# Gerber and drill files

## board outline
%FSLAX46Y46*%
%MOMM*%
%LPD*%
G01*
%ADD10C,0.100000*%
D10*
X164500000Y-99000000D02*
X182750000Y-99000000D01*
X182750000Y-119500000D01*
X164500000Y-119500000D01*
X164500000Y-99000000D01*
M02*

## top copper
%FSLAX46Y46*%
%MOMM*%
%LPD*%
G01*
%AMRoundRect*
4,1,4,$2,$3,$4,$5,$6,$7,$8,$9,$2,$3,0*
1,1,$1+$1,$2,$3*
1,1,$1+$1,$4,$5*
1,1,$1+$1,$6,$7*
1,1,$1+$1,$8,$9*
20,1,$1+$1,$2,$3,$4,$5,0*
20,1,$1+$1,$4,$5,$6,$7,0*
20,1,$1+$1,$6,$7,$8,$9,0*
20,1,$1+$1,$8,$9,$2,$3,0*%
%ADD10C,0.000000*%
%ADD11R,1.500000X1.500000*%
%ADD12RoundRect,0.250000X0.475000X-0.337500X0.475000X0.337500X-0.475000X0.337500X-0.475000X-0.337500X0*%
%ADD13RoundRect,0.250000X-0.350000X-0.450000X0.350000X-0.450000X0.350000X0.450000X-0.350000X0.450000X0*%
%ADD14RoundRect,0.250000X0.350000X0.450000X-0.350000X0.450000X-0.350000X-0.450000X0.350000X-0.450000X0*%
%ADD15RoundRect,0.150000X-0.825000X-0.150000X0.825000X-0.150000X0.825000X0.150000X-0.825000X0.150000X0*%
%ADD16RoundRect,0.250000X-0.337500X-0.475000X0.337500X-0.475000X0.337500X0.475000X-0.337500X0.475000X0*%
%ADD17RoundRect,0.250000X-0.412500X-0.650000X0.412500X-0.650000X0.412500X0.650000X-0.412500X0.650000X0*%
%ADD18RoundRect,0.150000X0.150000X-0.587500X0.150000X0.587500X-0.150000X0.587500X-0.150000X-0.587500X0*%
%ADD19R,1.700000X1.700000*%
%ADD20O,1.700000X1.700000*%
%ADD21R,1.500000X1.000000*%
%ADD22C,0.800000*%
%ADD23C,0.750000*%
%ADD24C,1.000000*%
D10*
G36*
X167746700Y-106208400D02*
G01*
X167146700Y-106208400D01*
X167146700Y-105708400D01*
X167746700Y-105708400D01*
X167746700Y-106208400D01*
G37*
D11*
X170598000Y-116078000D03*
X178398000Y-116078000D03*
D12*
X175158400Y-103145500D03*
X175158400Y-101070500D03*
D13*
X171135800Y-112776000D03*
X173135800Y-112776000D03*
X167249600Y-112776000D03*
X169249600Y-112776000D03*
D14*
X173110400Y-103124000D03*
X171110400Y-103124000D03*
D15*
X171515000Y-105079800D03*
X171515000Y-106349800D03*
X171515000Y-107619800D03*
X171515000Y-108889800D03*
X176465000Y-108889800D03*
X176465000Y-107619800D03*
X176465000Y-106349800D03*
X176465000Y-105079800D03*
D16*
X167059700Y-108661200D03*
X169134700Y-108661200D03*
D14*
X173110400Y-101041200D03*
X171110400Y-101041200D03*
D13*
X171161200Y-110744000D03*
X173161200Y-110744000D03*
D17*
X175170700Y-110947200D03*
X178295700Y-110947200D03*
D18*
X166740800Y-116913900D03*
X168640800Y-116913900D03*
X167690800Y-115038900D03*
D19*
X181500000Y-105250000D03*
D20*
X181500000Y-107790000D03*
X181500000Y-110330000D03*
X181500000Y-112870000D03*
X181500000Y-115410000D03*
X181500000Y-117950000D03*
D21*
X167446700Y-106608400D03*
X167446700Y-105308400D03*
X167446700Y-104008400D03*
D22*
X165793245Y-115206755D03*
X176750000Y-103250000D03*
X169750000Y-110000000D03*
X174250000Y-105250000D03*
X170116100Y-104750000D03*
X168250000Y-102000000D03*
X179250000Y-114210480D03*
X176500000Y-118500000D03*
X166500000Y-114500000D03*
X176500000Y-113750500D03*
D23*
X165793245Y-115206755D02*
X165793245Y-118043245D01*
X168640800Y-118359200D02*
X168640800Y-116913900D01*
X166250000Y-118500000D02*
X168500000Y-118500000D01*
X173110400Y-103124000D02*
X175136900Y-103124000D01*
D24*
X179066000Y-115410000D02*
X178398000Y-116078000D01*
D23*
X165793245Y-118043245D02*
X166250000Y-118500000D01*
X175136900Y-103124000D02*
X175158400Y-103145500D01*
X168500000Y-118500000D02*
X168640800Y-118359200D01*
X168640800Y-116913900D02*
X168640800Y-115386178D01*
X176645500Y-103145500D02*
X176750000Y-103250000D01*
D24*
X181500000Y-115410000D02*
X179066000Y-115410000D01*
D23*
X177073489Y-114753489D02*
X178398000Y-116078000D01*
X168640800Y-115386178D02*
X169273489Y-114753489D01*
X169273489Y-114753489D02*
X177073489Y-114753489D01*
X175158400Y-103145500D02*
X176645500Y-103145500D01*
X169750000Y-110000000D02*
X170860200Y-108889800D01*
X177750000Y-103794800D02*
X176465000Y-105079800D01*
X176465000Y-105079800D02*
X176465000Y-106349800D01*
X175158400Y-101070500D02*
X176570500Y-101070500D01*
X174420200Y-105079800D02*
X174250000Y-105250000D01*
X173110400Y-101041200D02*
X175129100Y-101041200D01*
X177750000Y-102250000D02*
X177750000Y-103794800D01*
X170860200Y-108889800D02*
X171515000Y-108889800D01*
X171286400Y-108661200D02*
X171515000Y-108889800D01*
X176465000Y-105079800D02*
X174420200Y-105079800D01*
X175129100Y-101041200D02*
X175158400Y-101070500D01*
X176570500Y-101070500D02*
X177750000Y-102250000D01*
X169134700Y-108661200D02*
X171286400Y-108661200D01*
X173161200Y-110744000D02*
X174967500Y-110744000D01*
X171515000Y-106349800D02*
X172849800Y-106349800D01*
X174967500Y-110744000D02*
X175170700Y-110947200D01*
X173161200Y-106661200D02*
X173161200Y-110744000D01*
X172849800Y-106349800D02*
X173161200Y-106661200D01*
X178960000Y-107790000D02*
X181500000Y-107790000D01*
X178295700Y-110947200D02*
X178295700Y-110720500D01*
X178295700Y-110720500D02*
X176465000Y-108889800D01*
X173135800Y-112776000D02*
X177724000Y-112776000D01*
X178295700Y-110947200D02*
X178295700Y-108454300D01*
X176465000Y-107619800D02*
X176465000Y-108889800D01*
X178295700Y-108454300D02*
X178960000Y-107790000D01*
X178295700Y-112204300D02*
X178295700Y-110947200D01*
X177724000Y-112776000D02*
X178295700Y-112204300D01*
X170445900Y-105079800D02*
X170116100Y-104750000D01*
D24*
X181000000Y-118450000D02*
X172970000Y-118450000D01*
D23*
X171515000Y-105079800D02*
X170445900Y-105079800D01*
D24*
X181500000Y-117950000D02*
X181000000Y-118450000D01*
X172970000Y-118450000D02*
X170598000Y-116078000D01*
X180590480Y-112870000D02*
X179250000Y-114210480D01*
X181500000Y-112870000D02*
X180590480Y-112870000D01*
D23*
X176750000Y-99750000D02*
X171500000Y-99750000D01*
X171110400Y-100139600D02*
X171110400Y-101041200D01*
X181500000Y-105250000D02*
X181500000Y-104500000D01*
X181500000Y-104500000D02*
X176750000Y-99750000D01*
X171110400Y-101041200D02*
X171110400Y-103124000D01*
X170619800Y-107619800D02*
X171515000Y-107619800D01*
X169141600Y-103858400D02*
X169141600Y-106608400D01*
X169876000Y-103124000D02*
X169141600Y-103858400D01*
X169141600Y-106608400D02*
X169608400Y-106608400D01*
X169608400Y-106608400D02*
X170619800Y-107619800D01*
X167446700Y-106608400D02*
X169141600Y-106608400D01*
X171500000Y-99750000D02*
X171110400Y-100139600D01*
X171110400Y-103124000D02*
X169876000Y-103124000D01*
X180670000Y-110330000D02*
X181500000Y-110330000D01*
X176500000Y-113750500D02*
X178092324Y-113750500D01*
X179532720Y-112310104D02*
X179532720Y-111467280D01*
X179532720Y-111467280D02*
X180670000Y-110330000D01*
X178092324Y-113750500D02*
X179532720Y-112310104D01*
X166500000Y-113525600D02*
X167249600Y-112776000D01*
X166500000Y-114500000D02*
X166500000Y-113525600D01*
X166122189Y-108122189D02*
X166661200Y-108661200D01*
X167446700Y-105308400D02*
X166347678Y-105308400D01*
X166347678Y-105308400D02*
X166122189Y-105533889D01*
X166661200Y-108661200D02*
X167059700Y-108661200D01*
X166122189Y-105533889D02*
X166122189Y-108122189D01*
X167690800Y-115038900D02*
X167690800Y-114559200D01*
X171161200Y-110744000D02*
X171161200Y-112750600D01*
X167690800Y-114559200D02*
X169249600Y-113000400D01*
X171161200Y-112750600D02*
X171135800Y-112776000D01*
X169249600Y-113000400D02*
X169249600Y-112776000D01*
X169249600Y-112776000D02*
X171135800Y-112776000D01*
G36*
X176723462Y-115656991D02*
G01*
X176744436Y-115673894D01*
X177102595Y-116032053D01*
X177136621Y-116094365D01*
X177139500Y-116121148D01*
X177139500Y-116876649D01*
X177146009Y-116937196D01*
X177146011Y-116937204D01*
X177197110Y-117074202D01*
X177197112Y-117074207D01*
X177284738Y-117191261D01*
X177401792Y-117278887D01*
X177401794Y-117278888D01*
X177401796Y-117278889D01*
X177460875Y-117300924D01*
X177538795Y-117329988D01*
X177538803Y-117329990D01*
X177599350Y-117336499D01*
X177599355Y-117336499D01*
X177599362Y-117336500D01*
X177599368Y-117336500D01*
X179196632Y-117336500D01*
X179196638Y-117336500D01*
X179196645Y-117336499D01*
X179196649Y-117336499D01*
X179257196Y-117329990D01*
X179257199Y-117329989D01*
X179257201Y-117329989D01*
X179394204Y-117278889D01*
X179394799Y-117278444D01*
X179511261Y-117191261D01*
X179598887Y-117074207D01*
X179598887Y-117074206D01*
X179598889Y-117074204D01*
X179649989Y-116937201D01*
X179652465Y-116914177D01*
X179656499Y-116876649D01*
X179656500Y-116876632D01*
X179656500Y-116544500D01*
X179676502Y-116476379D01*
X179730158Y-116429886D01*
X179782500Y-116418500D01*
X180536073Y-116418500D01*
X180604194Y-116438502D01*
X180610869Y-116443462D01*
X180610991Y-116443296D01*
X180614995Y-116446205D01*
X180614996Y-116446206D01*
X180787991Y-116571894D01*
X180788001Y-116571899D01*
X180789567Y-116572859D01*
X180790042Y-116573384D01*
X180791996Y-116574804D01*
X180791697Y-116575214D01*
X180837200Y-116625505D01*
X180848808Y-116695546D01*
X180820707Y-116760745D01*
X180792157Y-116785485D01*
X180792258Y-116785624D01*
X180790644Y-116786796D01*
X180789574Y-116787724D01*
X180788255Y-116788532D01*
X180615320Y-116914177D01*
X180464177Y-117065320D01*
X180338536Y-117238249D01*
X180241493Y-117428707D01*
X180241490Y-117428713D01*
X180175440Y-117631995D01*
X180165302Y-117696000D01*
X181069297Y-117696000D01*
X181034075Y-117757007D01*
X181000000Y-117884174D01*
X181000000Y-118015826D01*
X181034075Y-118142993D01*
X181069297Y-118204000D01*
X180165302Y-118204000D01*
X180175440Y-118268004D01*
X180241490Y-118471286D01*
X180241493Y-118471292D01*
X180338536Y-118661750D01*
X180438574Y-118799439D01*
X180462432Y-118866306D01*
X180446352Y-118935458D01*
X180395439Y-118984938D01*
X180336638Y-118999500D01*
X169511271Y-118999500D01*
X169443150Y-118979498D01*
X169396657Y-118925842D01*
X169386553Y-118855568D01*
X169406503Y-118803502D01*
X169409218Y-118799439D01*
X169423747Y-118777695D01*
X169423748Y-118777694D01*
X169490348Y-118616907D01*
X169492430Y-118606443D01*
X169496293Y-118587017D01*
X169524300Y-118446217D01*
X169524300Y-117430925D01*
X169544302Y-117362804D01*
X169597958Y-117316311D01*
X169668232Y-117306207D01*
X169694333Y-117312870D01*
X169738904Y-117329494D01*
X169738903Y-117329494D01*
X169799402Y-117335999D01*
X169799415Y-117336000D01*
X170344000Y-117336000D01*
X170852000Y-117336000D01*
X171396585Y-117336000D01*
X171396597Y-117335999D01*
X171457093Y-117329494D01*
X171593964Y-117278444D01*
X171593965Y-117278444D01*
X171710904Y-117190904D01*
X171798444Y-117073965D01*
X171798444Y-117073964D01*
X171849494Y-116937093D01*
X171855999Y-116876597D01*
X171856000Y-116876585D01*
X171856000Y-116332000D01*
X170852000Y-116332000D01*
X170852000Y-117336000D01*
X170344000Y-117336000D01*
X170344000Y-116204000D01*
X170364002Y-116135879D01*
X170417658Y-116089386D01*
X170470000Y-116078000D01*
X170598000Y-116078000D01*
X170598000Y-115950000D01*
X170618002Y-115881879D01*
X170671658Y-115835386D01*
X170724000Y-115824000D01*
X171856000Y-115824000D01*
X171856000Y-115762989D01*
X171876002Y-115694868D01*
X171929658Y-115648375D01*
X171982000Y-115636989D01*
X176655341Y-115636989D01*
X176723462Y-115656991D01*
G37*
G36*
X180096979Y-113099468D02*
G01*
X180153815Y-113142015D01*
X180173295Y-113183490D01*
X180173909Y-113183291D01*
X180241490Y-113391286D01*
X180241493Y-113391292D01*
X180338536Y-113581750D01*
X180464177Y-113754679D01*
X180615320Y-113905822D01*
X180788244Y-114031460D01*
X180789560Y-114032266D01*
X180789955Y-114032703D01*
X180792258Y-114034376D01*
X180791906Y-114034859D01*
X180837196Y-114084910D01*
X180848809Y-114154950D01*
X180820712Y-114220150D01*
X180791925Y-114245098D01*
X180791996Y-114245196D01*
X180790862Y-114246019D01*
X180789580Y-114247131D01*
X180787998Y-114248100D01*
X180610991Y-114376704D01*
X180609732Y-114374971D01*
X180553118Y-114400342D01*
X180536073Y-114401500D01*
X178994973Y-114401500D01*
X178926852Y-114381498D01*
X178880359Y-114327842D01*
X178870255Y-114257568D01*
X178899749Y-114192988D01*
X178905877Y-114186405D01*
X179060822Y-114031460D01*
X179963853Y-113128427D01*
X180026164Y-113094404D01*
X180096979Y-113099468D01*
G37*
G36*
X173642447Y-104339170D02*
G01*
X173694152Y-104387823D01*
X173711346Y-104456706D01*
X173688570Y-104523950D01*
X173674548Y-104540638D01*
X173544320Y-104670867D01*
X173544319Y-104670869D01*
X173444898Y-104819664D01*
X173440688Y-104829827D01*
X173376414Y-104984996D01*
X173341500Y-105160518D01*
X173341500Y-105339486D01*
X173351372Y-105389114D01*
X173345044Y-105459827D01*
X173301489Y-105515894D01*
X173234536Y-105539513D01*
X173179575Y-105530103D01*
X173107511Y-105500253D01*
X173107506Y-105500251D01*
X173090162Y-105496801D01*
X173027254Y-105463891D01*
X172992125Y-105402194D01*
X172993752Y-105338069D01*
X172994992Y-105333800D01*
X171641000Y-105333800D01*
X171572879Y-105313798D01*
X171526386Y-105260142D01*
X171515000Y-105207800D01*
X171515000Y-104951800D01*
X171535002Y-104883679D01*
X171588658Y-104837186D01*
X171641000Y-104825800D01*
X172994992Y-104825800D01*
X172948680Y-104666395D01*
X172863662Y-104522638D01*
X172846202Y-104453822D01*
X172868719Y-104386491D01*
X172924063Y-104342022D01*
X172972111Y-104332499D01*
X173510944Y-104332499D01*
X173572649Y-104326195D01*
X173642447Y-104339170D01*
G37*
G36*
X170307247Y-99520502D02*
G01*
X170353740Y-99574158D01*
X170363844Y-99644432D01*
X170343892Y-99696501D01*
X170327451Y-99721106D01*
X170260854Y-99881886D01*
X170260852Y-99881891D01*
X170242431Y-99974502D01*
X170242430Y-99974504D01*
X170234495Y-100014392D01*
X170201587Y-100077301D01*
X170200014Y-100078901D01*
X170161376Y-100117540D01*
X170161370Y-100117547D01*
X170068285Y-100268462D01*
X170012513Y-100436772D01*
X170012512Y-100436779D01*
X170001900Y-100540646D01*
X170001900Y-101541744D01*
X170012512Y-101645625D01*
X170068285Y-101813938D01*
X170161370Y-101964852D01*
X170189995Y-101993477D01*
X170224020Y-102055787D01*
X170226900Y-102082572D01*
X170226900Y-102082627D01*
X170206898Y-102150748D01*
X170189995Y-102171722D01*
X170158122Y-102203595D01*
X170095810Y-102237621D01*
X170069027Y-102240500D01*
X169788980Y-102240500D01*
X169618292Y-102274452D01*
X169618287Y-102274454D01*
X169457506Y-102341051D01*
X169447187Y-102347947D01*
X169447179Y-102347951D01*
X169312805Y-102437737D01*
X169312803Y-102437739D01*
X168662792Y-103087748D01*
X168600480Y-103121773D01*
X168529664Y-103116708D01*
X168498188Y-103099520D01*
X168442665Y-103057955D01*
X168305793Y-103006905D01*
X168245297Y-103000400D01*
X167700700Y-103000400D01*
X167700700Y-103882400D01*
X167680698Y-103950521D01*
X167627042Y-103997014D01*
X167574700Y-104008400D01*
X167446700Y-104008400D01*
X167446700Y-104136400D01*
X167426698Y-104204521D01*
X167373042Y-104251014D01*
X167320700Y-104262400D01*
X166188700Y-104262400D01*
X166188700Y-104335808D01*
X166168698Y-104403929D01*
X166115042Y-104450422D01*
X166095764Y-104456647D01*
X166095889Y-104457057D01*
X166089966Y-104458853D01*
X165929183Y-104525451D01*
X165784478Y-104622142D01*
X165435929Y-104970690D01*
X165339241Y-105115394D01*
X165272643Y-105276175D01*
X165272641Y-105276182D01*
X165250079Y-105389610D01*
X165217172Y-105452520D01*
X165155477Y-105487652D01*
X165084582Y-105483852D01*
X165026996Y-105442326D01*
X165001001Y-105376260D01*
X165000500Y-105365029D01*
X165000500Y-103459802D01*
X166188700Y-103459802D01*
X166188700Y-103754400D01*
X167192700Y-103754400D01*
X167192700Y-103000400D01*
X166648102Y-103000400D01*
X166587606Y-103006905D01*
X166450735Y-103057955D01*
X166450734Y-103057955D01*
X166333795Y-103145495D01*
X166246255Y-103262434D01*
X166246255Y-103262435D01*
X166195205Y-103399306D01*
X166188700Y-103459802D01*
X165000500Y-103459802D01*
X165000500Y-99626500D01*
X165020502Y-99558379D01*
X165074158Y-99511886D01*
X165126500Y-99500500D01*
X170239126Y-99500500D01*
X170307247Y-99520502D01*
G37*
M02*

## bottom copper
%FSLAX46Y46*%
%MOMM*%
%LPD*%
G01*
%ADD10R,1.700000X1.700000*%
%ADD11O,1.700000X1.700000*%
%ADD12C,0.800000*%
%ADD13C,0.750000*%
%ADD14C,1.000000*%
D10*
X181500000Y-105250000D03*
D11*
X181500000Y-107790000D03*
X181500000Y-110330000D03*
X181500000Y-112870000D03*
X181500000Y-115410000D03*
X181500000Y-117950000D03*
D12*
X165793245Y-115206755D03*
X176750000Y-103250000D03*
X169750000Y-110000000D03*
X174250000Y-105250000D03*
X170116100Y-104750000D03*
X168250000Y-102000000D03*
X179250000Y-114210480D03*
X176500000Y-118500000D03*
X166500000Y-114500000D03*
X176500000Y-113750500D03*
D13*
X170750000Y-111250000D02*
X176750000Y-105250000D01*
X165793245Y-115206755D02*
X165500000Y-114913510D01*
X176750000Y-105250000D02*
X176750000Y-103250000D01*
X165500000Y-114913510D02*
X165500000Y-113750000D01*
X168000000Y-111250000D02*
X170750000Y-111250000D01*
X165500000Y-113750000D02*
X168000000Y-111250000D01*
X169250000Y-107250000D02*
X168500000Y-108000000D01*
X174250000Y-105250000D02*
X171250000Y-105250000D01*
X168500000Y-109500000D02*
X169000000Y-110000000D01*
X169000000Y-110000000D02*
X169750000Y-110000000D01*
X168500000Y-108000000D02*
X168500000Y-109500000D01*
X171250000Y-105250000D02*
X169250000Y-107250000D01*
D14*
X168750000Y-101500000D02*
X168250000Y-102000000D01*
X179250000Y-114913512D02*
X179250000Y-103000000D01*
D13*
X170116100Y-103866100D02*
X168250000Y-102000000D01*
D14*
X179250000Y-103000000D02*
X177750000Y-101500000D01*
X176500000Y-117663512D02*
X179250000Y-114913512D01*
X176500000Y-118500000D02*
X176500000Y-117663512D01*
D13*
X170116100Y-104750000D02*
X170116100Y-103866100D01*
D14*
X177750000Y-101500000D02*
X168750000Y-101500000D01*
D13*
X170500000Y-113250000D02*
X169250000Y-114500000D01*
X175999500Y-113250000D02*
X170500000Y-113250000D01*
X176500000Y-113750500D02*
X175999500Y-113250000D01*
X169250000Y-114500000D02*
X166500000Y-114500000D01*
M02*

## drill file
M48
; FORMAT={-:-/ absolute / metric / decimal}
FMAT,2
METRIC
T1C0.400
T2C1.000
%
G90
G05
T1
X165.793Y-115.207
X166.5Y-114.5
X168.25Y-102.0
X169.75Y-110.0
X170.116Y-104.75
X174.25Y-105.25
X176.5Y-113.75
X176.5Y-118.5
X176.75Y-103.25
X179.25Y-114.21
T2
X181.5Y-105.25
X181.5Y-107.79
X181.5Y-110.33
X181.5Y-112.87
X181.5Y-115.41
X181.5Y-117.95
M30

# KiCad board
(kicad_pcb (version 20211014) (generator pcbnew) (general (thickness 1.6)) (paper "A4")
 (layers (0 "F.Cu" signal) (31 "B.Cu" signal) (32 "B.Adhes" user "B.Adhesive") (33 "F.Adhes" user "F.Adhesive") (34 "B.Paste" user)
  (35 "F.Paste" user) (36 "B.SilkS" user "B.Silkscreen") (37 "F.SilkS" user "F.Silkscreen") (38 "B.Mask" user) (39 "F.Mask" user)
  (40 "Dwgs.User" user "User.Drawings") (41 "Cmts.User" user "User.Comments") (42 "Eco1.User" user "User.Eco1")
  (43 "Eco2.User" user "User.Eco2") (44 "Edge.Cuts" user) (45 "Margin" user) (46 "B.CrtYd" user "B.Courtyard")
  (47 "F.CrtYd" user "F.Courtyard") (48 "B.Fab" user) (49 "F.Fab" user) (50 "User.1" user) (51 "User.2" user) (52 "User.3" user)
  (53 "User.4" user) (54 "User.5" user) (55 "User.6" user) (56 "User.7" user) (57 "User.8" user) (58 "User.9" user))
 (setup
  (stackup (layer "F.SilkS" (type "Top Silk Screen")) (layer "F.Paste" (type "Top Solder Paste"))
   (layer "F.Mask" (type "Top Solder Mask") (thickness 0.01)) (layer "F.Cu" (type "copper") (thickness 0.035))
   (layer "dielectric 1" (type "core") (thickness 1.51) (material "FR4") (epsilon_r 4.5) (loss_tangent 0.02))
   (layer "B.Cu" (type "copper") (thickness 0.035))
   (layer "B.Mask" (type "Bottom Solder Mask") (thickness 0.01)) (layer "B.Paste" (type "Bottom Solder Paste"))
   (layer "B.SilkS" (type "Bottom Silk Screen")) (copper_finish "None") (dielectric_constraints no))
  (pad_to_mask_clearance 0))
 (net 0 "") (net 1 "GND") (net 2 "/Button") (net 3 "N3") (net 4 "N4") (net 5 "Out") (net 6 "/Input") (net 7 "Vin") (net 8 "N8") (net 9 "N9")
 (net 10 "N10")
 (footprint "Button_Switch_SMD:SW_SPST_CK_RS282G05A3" (layer "F.Cu") (at 174.498 116.078)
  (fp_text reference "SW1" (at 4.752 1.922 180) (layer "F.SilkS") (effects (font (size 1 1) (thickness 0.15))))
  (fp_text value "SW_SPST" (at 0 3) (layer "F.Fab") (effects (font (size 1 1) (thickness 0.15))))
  (pad "1" smd rect locked (at -3.9 0) (size 1.5 1.5) (layers "F.Cu" "F.Paste" "F.Mask") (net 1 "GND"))
  (pad "2" smd rect locked (at 3.9 0) (size 1.5 1.5) (layers "F.Cu" "F.Paste" "F.Mask") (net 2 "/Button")))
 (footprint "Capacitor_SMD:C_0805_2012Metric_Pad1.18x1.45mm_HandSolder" (layer "F.Cu") (at 175.1584 102.108 90)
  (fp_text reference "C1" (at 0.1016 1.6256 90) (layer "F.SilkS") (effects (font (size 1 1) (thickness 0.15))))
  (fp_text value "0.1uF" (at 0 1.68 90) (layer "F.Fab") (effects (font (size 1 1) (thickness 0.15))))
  (pad "1" smd roundrect locked (at -1.0375 0 90) (size 1.175 1.45) (layers "F.Cu" "F.Paste" "F.Mask") (roundrect_rratio 0.212766)
   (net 2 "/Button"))
  (pad "2" smd roundrect locked (at 1.0375 0 90) (size 1.175 1.45) (layers "F.Cu" "F.Paste" "F.Mask") (roundrect_rratio 0.212766)
   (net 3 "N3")))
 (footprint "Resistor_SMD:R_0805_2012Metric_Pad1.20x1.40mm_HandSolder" (layer "F.Cu") (at 172.1358 112.776)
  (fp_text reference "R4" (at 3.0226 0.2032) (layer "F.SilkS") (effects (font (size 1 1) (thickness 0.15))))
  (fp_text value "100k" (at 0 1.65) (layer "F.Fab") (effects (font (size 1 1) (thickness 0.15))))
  (pad "1" smd roundrect locked (at -1 0) (size 1.2 1.4) (layers "F.Cu" "F.Paste" "F.Mask") (roundrect_rratio 0.208333) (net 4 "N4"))
  (pad "2" smd roundrect locked (at 1 0) (size 1.2 1.4) (layers "F.Cu" "F.Paste" "F.Mask") (roundrect_rratio 0.208333) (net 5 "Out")))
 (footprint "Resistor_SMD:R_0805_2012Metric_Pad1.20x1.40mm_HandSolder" (layer "F.Cu") (at 168.2496 112.776)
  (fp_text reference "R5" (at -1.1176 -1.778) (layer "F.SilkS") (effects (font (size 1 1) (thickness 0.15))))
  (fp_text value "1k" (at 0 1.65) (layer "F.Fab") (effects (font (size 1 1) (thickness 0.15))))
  (pad "1" smd roundrect locked (at -1 0) (size 1.2 1.4) (layers "F.Cu" "F.Paste" "F.Mask") (roundrect_rratio 0.208333) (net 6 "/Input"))
  (pad "2" smd roundrect locked (at 1 0) (size 1.2 1.4) (layers "F.Cu" "F.Paste" "F.Mask") (roundrect_rratio 0.208333) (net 4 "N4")))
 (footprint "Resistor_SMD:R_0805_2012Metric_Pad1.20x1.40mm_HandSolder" (layer "F.Cu") (at 172.1104 103.124 180)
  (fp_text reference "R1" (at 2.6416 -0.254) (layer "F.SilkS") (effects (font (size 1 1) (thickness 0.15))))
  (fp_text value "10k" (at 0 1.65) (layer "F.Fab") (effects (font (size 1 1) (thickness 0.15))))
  (pad "1" smd roundrect locked (at -1 0 180) (size 1.2 1.4) (layers "F.Cu" "F.Paste" "F.Mask") (roundrect_rratio 0.208333)
   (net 2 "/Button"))
  (pad "2" smd roundrect locked (at 1 0 180) (size 1.2 1.4) (layers "F.Cu" "F.Paste" "F.Mask") (roundrect_rratio 0.208333) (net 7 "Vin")))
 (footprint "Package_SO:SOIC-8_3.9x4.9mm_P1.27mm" (layer "F.Cu") (at 173.99 106.9848)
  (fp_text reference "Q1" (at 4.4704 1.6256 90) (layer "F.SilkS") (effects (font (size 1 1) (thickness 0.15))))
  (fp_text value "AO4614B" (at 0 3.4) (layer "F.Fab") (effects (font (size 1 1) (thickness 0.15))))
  (pad "1" smd roundrect locked (at -2.475 -1.905) (size 1.95 0.6) (layers "F.Cu" "F.Paste" "F.Mask") (roundrect_rratio 0.25) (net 1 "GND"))
  (pad "2" smd roundrect locked (at -2.475 -0.635) (size 1.95 0.6) (layers "F.Cu" "F.Paste" "F.Mask") (roundrect_rratio 0.25) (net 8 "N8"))
  (pad "3" smd roundrect locked (at -2.475 0.635) (size 1.95 0.6) (layers "F.Cu" "F.Paste" "F.Mask") (roundrect_rratio 0.25) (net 7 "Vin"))
  (pad "4" smd roundrect locked (at -2.475 1.905) (size 1.95 0.6) (layers "F.Cu" "F.Paste" "F.Mask") (roundrect_rratio 0.25) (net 3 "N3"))
  (pad "5" smd roundrect locked (at 2.475 1.905) (size 1.95 0.6) (layers "F.Cu" "F.Paste" "F.Mask") (roundrect_rratio 0.25) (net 5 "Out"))
  (pad "6" smd roundrect locked (at 2.475 0.635) (size 1.95 0.6) (layers "F.Cu" "F.Paste" "F.Mask") (roundrect_rratio 0.25) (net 5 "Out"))
  (pad "7" smd roundrect locked (at 2.475 -0.635) (size 1.95 0.6) (layers "F.Cu" "F.Paste" "F.Mask") (roundrect_rratio 0.25) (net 3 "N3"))
  (pad "8" smd roundrect locked (at 2.475 -1.905) (size 1.95 0.6) (layers "F.Cu" "F.Paste" "F.Mask") (roundrect_rratio 0.25) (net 3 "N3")))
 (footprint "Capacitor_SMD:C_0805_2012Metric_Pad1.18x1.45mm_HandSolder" (layer "F.Cu") (at 168.0972 108.6612)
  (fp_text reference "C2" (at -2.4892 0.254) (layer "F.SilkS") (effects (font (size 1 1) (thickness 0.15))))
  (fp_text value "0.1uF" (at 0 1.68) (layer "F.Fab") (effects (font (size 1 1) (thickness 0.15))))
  (pad "1" smd roundrect locked (at -1.0375 0) (size 1.175 1.45) (layers "F.Cu" "F.Paste" "F.Mask") (roundrect_rratio 0.212766) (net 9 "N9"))
  (pad "2" smd roundrect locked (at 1.0375 0) (size 1.175 1.45) (layers "F.Cu" "F.Paste" "F.Mask") (roundrect_rratio 0.212766) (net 3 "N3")))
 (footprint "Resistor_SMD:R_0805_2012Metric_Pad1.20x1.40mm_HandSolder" (layer "F.Cu") (at 172.1104 101.0412 180)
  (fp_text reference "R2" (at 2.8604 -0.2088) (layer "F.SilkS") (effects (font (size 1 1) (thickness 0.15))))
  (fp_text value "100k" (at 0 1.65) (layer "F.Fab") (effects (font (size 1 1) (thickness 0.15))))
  (pad "1" smd roundrect locked (at -1 0 180) (size 1.2 1.4) (layers "F.Cu" "F.Paste" "F.Mask") (roundrect_rratio 0.208333) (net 3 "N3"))
  (pad "2" smd roundrect locked (at 1 0 180) (size 1.2 1.4) (layers "F.Cu" "F.Paste" "F.Mask") (roundrect_rratio 0.208333) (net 7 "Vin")))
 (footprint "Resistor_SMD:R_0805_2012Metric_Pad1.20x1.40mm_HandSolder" (layer "F.Cu") (at 172.1612 110.744)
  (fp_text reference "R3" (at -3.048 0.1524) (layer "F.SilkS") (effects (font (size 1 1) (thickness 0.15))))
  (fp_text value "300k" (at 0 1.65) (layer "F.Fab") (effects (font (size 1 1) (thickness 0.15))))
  (pad "1" smd roundrect locked (at -1 0) (size 1.2 1.4) (layers "F.Cu" "F.Paste" "F.Mask") (roundrect_rratio 0.208333) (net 4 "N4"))
  (pad "2" smd roundrect locked (at 1 0) (size 1.2 1.4) (layers "F.Cu" "F.Paste" "F.Mask") (roundrect_rratio 0.208333) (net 8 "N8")))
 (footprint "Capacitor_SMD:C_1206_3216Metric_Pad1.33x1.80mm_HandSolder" (layer "F.Cu") (at 176.7332 110.9472)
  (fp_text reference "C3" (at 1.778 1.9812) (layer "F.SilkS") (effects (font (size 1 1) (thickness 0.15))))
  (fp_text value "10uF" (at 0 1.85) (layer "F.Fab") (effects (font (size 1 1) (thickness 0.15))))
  (pad "1" smd roundrect locked (at -1.5625 0) (size 1.325 1.8) (layers "F.Cu" "F.Paste" "F.Mask") (roundrect_rratio 0.188679) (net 8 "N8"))
  (pad "2" smd roundrect locked (at 1.5625 0) (size 1.325 1.8) (layers "F.Cu" "F.Paste" "F.Mask") (roundrect_rratio 0.188679) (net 5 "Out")))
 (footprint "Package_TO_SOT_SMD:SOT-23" (layer "F.Cu") (at 167.6908 115.9764 90)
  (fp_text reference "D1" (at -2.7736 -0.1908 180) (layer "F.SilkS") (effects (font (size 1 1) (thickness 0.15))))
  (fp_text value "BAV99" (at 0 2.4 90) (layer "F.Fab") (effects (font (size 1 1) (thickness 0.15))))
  (pad "1" smd roundrect locked (at -0.9375 -0.95 90) (size 1.475 0.6) (layers "F.Cu" "F.Paste" "F.Mask") (roundrect_rratio 0.25)
   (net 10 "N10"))
  (pad "2" smd roundrect locked (at -0.9375 0.95 90) (size 1.475 0.6) (layers "F.Cu" "F.Paste" "F.Mask") (roundrect_rratio 0.25)
   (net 2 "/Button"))
  (pad "3" smd roundrect locked (at 0.9375 0 90) (size 1.475 0.6) (layers "F.Cu" "F.Paste" "F.Mask") (roundrect_rratio 0.25) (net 4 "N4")))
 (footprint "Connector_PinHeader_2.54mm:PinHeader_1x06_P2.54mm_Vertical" (layer "F.Cu") (at 181.5 105.25)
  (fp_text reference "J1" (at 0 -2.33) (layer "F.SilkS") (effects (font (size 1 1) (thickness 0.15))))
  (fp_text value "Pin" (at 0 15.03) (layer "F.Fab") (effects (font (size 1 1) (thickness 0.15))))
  (pad "1" thru_hole rect locked (at 0 0) (size 1.7 1.7) (drill 1) (layers *.Cu *.Mask) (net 7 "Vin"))
  (pad "2" thru_hole oval locked (at 0 2.54) (size 1.7 1.7) (drill 1) (layers *.Cu *.Mask) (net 5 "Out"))
  (pad "3" thru_hole oval locked (at 0 5.08) (size 1.7 1.7) (drill 1) (layers *.Cu *.Mask) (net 6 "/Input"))
  (pad "4" thru_hole oval locked (at 0 7.62) (size 1.7 1.7) (drill 1) (layers *.Cu *.Mask) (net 1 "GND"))
  (pad "5" thru_hole oval locked (at 0 10.16) (size 1.7 1.7) (drill 1) (layers *.Cu *.Mask) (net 2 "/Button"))
  (pad "6" thru_hole oval locked (at 0 12.7) (size 1.7 1.7) (drill 1) (layers *.Cu *.Mask) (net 1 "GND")))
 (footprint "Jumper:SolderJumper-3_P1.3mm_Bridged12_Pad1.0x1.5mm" (layer "F.Cu") (at 167.4467 105.3084 90)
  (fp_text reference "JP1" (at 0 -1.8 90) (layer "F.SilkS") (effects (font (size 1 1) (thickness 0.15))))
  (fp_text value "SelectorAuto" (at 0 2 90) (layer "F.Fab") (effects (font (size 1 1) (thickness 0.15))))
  (fp_poly (pts (xy -0.9 -0.3) (xy -0.4 -0.3) (xy -0.4 0.3) (xy -0.9 0.3)) (layer "F.Cu") (width 0) (fill solid))
  (pad "1" smd rect locked (at -1.3 0 90) (size 1 1.5) (layers "F.Cu" "F.Mask") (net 7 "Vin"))
  (pad "2" smd rect locked (at 0 0 90) (size 1 1.5) (layers "F.Cu" "F.Mask") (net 9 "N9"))
  (pad "3" smd rect locked (at 1.3 0 90) (size 1 1.5) (layers "F.Cu" "F.Mask") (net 1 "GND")))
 (gr_rect (start 164.5 99) (end 182.75 119.5) (layer "Edge.Cuts") (width 0.1) (fill none))
 (segment (start 165.793245 115.206755) (end 165.793245 118.043245) (width 0.75) (layer "F.Cu") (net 2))
 (segment (start 168.6408 118.3592) (end 168.6408 116.9139) (width 0.75) (layer "F.Cu") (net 2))
 (segment (start 166.25 118.5) (end 168.5 118.5) (width 0.75) (layer "F.Cu") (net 2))
 (segment (start 173.1104 103.124) (end 175.1369 103.124) (width 0.75) (layer "F.Cu") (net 2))
 (segment (start 179.066 115.41) (end 178.398 116.078) (width 1) (layer "F.Cu") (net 2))
 (segment (start 165.793245 118.043245) (end 166.25 118.5) (width 0.75) (layer "F.Cu") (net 2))
 (segment (start 175.1369 103.124) (end 175.1584 103.1455) (width 0.75) (layer "F.Cu") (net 2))
 (segment (start 168.5 118.5) (end 168.6408 118.3592) (width 0.75) (layer "F.Cu") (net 2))
 (segment (start 168.6408 116.9139) (end 168.6408 115.386178) (width 0.75) (layer "F.Cu") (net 2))
 (segment (start 176.6455 103.1455) (end 176.75 103.25) (width 0.75) (layer "F.Cu") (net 2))
 (segment (start 181.5 115.41) (end 179.066 115.41) (width 1) (layer "F.Cu") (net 2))
 (segment (start 177.073489 114.753489) (end 178.398 116.078) (width 0.75) (layer "F.Cu") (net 2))
 (segment (start 168.6408 115.386178) (end 169.273489 114.753489) (width 0.75) (layer "F.Cu") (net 2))
 (segment (start 169.273489 114.753489) (end 177.073489 114.753489) (width 0.75) (layer "F.Cu") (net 2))
 (segment (start 175.1584 103.1455) (end 176.6455 103.1455) (width 0.75) (layer "F.Cu") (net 2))
 (via (at 165.793245 115.206755) (size 0.8) (drill 0.4) (layers "F.Cu" "B.Cu") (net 2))
 (via (at 176.75 103.25) (size 0.8) (drill 0.4) (layers "F.Cu" "B.Cu") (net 2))
 (segment (start 170.75 111.25) (end 176.75 105.25) (width 0.75) (layer "B.Cu") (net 2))
 (segment (start 165.793245 115.206755) (end 165.5 114.91351) (width 0.75) (layer "B.Cu") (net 2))
 (segment (start 176.75 105.25) (end 176.75 103.25) (width 0.75) (layer "B.Cu") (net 2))
 (segment (start 165.5 114.91351) (end 165.5 113.75) (width 0.75) (layer "B.Cu") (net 2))
 (segment (start 168 111.25) (end 170.75 111.25) (width 0.75) (layer "B.Cu") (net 2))
 (segment (start 165.5 113.75) (end 168 111.25) (width 0.75) (layer "B.Cu") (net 2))
 (segment (start 169.75 110) (end 170.8602 108.8898) (width 0.75) (layer "F.Cu") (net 3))
 (segment (start 177.75 103.7948) (end 176.465 105.0798) (width 0.75) (layer "F.Cu") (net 3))
 (segment (start 176.465 105.0798) (end 176.465 106.3498) (width 0.75) (layer "F.Cu") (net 3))
 (segment (start 175.1584 101.0705) (end 176.5705 101.0705) (width 0.75) (layer "F.Cu") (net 3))
 (segment (start 174.4202 105.0798) (end 174.25 105.25) (width 0.75) (layer "F.Cu") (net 3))
 (segment (start 173.1104 101.0412) (end 175.1291 101.0412) (width 0.75) (layer "F.Cu") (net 3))
 (segment (start 177.75 102.25) (end 177.75 103.7948) (width 0.75) (layer "F.Cu") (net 3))
 (segment (start 170.8602 108.8898) (end 171.515 108.8898) (width 0.75) (layer "F.Cu") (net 3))
 (segment (start 171.2864 108.6612) (end 171.515 108.8898) (width 0.75) (layer "F.Cu") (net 3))
 (segment (start 176.465 105.0798) (end 174.4202 105.0798) (width 0.75) (layer "F.Cu") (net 3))
 (segment (start 175.1291 101.0412) (end 175.1584 101.0705) (width 0.75) (layer "F.Cu") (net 3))
 (segment (start 176.5705 101.0705) (end 177.75 102.25) (width 0.75) (layer "F.Cu") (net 3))
 (segment (start 169.1347 108.6612) (end 171.2864 108.6612) (width 0.75) (layer "F.Cu") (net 3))
 (via (at 169.75 110) (size 0.8) (drill 0.4) (layers "F.Cu" "B.Cu") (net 3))
 (via (at 174.25 105.25) (size 0.8) (drill 0.4) (layers "F.Cu" "B.Cu") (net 3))
 (segment (start 169.25 107.25) (end 168.5 108) (width 0.75) (layer "B.Cu") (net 3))
 (segment (start 174.25 105.25) (end 171.25 105.25) (width 0.75) (layer "B.Cu") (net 3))
 (segment (start 168.5 109.5) (end 169 110) (width 0.75) (layer "B.Cu") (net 3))
 (segment (start 169 110) (end 169.75 110) (width 0.75) (layer "B.Cu") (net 3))
 (segment (start 168.5 108) (end 168.5 109.5) (width 0.75) (layer "B.Cu") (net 3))
 (segment (start 171.25 105.25) (end 169.25 107.25) (width 0.75) (layer "B.Cu") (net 3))
 (segment (start 173.1612 110.744) (end 174.9675 110.744) (width 0.75) (layer "F.Cu") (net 8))
 (segment (start 171.515 106.3498) (end 172.8498 106.3498) (width 0.75) (layer "F.Cu") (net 8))
 (segment (start 174.9675 110.744) (end 175.1707 110.9472) (width 0.75) (layer "F.Cu") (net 8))
 (segment (start 173.1612 106.6612) (end 173.1612 110.744) (width 0.75) (layer "F.Cu") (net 8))
 (segment (start 172.8498 106.3498) (end 173.1612 106.6612) (width 0.75) (layer "F.Cu") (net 8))
 (segment (start 178.96 107.79) (end 181.5 107.79) (width 0.75) (layer "F.Cu") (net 5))
 (segment (start 178.2957 110.9472) (end 178.2957 110.7205) (width 0.75) (layer "F.Cu") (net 5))
 (segment (start 178.2957 110.7205) (end 176.465 108.8898) (width 0.75) (layer "F.Cu") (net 5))
 (segment (start 173.1358 112.776) (end 177.724 112.776) (width 0.75) (layer "F.Cu") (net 5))
 (segment (start 178.2957 110.9472) (end 178.2957 108.4543) (width 0.75) (layer "F.Cu") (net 5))
 (segment (start 176.465 107.6198) (end 176.465 108.8898) (width 0.75) (layer "F.Cu") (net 5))
 (segment (start 178.2957 108.4543) (end 178.96 107.79) (width 0.75) (layer "F.Cu") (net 5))
 (segment (start 178.2957 112.2043) (end 178.2957 110.9472) (width 0.75) (layer "F.Cu") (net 5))
 (segment (start 177.724 112.776) (end 178.2957 112.2043) (width 0.75) (layer "F.Cu") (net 5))
 (segment (start 170.4459 105.0798) (end 170.1161 104.75) (width 0.75) (layer "F.Cu") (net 1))
 (segment (start 181 118.45) (end 172.97 118.45) (width 1) (layer "F.Cu") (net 1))
 (segment (start 171.515 105.0798) (end 170.4459 105.0798) (width 0.75) (layer "F.Cu") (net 1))
 (segment (start 181.5 117.95) (end 181 118.45) (width 1) (layer "F.Cu") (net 1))
 (segment (start 172.97 118.45) (end 170.598 116.078) (width 1) (layer "F.Cu") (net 1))
 (segment (start 180.59048 112.87) (end 179.25 114.21048) (width 1) (layer "F.Cu") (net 1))
 (segment (start 181.5 112.87) (end 180.59048 112.87) (width 1) (layer "F.Cu") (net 1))
 (via (at 170.1161 104.75) (size 0.8) (drill 0.4) (layers "F.Cu" "B.Cu") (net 1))
 (via (at 168.25 102) (size 0.8) (drill 0.4) (layers "F.Cu" "B.Cu") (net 1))
 (via (at 179.25 114.21048) (size 0.8) (drill 0.4) (layers "F.Cu" "B.Cu") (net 1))
 (via (at 176.5 118.5) (size 0.8) (drill 0.4) (layers "F.Cu" "B.Cu") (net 1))
 (segment (start 168.75 101.5) (end 168.25 102) (width 1) (layer "B.Cu") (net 1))
 (segment (start 179.25 114.913512) (end 179.25 103) (width 1) (layer "B.Cu") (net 1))
 (segment (start 170.1161 103.8661) (end 168.25 102) (width 0.75) (layer "B.Cu") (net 1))
 (segment (start 179.25 103) (end 177.75 101.5) (width 1) (layer "B.Cu") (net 1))
 (segment (start 176.5 117.663512) (end 179.25 114.913512) (width 1) (layer "B.Cu") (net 1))
 (segment (start 176.5 118.5) (end 176.5 117.663512) (width 1) (layer "B.Cu") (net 1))
 (segment (start 170.1161 104.75) (end 170.1161 103.8661) (width 0.75) (layer "B.Cu") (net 1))
 (segment (start 177.75 101.5) (end 168.75 101.5) (width 1) (layer "B.Cu") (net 1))
 (segment (start 176.75 99.75) (end 171.5 99.75) (width 0.75) (layer "F.Cu") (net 7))
 (segment (start 171.1104 100.1396) (end 171.1104 101.0412) (width 0.75) (layer "F.Cu") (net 7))
 (segment (start 181.5 105.25) (end 181.5 104.5) (width 0.75) (layer "F.Cu") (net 7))
 (segment (start 181.5 104.5) (end 176.75 99.75) (width 0.75) (layer "F.Cu") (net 7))
 (segment (start 171.1104 101.0412) (end 171.1104 103.124) (width 0.75) (layer "F.Cu") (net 7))
 (segment (start 170.6198 107.6198) (end 171.515 107.6198) (width 0.75) (layer "F.Cu") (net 7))
 (segment (start 169.1416 103.8584) (end 169.1416 106.6084) (width 0.75) (layer "F.Cu") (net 7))
 (segment (start 169.876 103.124) (end 169.1416 103.8584) (width 0.75) (layer "F.Cu") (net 7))
 (segment (start 169.1416 106.6084) (end 169.6084 106.6084) (width 0.75) (layer "F.Cu") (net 7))
 (segment (start 169.6084 106.6084) (end 170.6198 107.6198) (width 0.75) (layer "F.Cu") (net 7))
 (segment (start 167.4467 106.6084) (end 169.1416 106.6084) (width 0.75) (layer "F.Cu") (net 7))
 (segment (start 171.5 99.75) (end 171.1104 100.1396) (width 0.75) (layer "F.Cu") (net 7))
 (segment (start 171.1104 103.124) (end 169.876 103.124) (width 0.75) (layer "F.Cu") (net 7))
 (segment (start 180.67 110.33) (end 181.5 110.33) (width 0.75) (layer "F.Cu") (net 6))
 (segment (start 176.5 113.7505) (end 178.092324 113.7505) (width 0.75) (layer "F.Cu") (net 6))
 (segment (start 179.53272 112.310104) (end 179.53272 111.46728) (width 0.75) (layer "F.Cu") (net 6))
 (segment (start 179.53272 111.46728) (end 180.67 110.33) (width 0.75) (layer "F.Cu") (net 6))
 (segment (start 178.092324 113.7505) (end 179.53272 112.310104) (width 0.75) (layer "F.Cu") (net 6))
 (segment (start 166.5 113.5256) (end 167.2496 112.776) (width 0.75) (layer "F.Cu") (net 6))
 (segment (start 166.5 114.5) (end 166.5 113.5256) (width 0.75) (layer "F.Cu") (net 6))
 (via (at 166.5 114.5) (size 0.8) (drill 0.4) (layers "F.Cu" "B.Cu") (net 6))
 (via (at 176.5 113.7505) (size 0.8) (drill 0.4) (layers "F.Cu" "B.Cu") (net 6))
 (segment (start 170.5 113.25) (end 169.25 114.5) (width 0.75) (layer "B.Cu") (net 6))
 (segment (start 175.9995 113.25) (end 170.5 113.25) (width 0.75) (layer "B.Cu") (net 6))
 (segment (start 176.5 113.7505) (end 175.9995 113.25) (width 0.75) (layer "B.Cu") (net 6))
 (segment (start 169.25 114.5) (end 166.5 114.5) (width 0.75) (layer "B.Cu") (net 6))
 (segment (start 166.122189 108.122189) (end 166.6612 108.6612) (width 0.75) (layer "F.Cu") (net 9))
 (segment (start 167.4467 105.3084) (end 166.347678 105.3084) (width 0.75) (layer "F.Cu") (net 9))
 (segment (start 166.347678 105.3084) (end 166.122189 105.533889) (width 0.75) (layer "F.Cu") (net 9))
 (segment (start 166.6612 108.6612) (end 167.0597 108.6612) (width 0.75) (layer "F.Cu") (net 9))
 (segment (start 166.122189 105.533889) (end 166.122189 108.122189) (width 0.75) (layer "F.Cu") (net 9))
 (segment (start 167.6908 115.0389) (end 167.6908 114.5592) (width 0.75) (layer "F.Cu") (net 4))
 (segment (start 171.1612 110.744) (end 171.1612 112.7506) (width 0.75) (layer "F.Cu") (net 4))
 (segment (start 167.6908 114.5592) (end 169.2496 113.0004) (width 0.75) (layer "F.Cu") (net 4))
 (segment (start 171.1612 112.7506) (end 171.1358 112.776) (width 0.75) (layer "F.Cu") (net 4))
 (segment (start 169.2496 113.0004) (end 169.2496 112.776) (width 0.75) (layer "F.Cu") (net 4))
 (segment (start 169.2496 112.776) (end 171.1358 112.776) (width 0.75) (layer "F.Cu") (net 4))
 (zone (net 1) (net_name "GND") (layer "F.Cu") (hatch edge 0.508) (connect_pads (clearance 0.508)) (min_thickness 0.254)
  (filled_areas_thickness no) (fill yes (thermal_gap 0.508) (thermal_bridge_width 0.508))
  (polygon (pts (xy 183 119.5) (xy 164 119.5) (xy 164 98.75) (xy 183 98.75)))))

